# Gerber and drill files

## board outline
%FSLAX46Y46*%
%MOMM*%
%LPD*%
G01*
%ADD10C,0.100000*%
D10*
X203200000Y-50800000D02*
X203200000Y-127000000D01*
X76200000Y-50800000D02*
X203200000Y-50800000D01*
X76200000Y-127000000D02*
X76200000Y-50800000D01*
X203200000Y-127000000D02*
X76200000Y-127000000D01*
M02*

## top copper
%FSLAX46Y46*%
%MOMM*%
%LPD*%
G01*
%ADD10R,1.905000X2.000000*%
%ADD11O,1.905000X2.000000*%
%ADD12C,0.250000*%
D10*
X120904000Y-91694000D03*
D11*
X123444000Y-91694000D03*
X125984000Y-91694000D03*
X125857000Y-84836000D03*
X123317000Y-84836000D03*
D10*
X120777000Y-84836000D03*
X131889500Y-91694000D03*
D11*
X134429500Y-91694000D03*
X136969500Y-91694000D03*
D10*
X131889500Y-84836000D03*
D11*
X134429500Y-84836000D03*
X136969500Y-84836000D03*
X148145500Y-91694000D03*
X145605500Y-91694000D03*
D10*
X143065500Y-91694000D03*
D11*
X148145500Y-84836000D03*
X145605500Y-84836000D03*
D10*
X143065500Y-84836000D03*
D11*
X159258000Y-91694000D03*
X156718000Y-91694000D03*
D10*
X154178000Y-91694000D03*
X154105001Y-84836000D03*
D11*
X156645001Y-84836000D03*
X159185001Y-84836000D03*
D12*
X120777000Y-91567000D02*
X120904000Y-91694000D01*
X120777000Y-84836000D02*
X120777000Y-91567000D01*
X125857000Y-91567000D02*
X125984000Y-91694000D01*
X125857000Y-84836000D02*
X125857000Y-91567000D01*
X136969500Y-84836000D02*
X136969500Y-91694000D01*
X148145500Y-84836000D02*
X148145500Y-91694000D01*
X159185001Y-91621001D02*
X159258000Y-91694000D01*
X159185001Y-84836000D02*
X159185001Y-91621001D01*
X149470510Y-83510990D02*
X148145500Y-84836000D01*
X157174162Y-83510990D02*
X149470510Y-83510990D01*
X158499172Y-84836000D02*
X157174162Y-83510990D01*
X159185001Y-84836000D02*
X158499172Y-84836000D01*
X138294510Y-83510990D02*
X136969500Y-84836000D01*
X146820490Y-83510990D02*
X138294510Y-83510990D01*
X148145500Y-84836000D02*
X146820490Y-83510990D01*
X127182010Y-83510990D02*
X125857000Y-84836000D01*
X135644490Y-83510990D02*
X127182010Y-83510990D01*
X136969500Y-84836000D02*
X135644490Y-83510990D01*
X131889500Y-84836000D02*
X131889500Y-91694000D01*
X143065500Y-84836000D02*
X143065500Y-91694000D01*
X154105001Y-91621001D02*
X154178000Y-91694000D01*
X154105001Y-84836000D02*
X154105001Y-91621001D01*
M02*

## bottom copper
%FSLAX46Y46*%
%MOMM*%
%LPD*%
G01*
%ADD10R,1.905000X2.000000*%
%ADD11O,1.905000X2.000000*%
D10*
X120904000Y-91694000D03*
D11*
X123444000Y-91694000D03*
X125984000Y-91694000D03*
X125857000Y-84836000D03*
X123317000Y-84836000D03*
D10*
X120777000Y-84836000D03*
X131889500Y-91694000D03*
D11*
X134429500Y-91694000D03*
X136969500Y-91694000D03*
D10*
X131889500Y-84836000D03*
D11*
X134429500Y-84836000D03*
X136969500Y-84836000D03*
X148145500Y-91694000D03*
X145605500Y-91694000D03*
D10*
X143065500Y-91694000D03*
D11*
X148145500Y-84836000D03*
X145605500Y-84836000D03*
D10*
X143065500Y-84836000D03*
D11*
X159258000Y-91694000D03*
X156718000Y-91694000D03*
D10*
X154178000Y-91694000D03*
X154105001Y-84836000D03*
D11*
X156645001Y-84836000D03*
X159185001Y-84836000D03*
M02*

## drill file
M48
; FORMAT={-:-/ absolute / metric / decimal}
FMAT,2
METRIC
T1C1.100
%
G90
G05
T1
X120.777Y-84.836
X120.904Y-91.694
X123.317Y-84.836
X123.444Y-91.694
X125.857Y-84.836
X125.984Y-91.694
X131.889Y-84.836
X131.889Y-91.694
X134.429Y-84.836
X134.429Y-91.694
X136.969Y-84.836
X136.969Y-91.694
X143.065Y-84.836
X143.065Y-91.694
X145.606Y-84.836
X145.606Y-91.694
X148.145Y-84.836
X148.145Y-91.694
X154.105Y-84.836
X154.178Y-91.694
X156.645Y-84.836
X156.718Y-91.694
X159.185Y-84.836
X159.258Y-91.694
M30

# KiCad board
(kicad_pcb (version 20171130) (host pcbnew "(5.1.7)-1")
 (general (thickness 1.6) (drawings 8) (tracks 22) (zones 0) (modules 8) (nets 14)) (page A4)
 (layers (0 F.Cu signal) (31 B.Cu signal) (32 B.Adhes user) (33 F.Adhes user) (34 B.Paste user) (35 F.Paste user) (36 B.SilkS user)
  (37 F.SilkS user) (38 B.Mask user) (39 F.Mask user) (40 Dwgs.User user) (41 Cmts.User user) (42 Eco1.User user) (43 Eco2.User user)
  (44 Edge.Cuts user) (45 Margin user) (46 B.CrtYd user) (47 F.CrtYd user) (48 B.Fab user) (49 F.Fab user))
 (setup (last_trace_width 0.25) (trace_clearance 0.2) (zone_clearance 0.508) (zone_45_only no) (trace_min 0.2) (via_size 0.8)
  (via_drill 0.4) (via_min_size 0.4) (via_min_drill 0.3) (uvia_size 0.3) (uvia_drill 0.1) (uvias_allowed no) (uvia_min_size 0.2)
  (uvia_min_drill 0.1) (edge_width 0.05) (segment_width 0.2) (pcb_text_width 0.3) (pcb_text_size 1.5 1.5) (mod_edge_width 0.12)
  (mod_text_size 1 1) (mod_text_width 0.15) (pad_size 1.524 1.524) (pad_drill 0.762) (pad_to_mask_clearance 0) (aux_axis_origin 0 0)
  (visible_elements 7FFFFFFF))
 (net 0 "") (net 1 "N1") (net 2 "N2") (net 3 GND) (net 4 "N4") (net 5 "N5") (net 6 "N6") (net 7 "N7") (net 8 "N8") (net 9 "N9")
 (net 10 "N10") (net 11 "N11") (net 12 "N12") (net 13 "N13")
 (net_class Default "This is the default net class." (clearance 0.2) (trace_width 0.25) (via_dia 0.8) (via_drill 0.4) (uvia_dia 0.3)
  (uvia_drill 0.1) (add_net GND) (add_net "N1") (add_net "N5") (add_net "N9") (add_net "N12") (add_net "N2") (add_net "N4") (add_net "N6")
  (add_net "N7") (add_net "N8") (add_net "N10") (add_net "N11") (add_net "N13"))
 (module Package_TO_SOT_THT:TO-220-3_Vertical (layer F.Cu) (at 120.904 91.694)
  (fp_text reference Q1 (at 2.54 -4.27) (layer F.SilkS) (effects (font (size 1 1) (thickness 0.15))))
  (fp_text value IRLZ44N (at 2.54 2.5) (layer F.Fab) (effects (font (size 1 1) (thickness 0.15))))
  (pad 1 thru_hole rect (at 0 0) (size 1.905 2) (drill 1.1) (layers *.Cu *.Mask) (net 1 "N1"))
  (pad 2 thru_hole oval (at 2.54 0) (size 1.905 2) (drill 1.1) (layers *.Cu *.Mask) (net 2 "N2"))
  (pad 3 thru_hole oval (at 5.08 0) (size 1.905 2) (drill 1.1) (layers *.Cu *.Mask) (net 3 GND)))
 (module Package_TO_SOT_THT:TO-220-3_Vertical (layer F.Cu) (at 120.777 84.836)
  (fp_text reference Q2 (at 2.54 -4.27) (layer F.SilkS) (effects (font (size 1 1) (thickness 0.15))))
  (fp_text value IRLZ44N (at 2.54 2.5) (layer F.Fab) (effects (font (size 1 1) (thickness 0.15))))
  (pad 3 thru_hole oval (at 5.08 0) (size 1.905 2) (drill 1.1) (layers *.Cu *.Mask) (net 3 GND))
  (pad 2 thru_hole oval (at 2.54 0) (size 1.905 2) (drill 1.1) (layers *.Cu *.Mask) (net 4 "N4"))
  (pad 1 thru_hole rect (at 0 0) (size 1.905 2) (drill 1.1) (layers *.Cu *.Mask) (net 1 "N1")))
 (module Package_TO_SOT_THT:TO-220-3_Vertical (layer F.Cu) (at 131.8895 91.694)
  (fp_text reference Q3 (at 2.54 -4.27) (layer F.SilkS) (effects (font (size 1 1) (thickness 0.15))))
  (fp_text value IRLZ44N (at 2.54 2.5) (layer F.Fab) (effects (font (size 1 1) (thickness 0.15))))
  (pad 1 thru_hole rect (at 0 0) (size 1.905 2) (drill 1.1) (layers *.Cu *.Mask) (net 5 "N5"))
  (pad 2 thru_hole oval (at 2.54 0) (size 1.905 2) (drill 1.1) (layers *.Cu *.Mask) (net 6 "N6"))
  (pad 3 thru_hole oval (at 5.08 0) (size 1.905 2) (drill 1.1) (layers *.Cu *.Mask) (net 3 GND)))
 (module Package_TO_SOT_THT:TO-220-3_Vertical (layer F.Cu) (at 131.8895 84.836)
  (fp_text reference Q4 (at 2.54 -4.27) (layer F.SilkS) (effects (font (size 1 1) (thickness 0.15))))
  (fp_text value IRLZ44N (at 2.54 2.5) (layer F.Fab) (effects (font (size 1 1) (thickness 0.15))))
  (pad 1 thru_hole rect (at 0 0) (size 1.905 2) (drill 1.1) (layers *.Cu *.Mask) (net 5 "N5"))
  (pad 2 thru_hole oval (at 2.54 0) (size 1.905 2) (drill 1.1) (layers *.Cu *.Mask) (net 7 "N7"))
  (pad 3 thru_hole oval (at 5.08 0) (size 1.905 2) (drill 1.1) (layers *.Cu *.Mask) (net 3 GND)))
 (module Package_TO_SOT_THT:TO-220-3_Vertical (layer F.Cu) (at 143.0655 91.694)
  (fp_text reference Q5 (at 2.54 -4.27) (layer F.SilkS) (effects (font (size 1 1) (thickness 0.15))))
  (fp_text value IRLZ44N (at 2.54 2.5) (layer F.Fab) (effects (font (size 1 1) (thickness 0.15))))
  (pad 3 thru_hole oval (at 5.08 0) (size 1.905 2) (drill 1.1) (layers *.Cu *.Mask) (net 3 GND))
  (pad 2 thru_hole oval (at 2.54 0) (size 1.905 2) (drill 1.1) (layers *.Cu *.Mask) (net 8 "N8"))
  (pad 1 thru_hole rect (at 0 0) (size 1.905 2) (drill 1.1) (layers *.Cu *.Mask) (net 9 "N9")))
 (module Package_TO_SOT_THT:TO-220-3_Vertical (layer F.Cu) (at 143.0655 84.836)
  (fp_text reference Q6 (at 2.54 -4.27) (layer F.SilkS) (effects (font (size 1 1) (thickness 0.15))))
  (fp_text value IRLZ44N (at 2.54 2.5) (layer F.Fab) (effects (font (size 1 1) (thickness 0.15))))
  (pad 3 thru_hole oval (at 5.08 0) (size 1.905 2) (drill 1.1) (layers *.Cu *.Mask) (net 3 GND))
  (pad 2 thru_hole oval (at 2.54 0) (size 1.905 2) (drill 1.1) (layers *.Cu *.Mask) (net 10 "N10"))
  (pad 1 thru_hole rect (at 0 0) (size 1.905 2) (drill 1.1) (layers *.Cu *.Mask) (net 9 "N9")))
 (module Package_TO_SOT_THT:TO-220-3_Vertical (layer F.Cu) (at 154.178 91.694)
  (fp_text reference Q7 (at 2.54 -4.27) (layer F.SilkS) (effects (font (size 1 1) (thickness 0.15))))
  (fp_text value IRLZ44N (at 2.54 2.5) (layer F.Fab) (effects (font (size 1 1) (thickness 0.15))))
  (pad 3 thru_hole oval (at 5.08 0) (size 1.905 2) (drill 1.1) (layers *.Cu *.Mask) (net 3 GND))
  (pad 2 thru_hole oval (at 2.54 0) (size 1.905 2) (drill 1.1) (layers *.Cu *.Mask) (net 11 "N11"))
  (pad 1 thru_hole rect (at 0 0) (size 1.905 2) (drill 1.1) (layers *.Cu *.Mask) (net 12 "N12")))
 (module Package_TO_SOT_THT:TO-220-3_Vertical (layer F.Cu) (at 154.105001 84.836)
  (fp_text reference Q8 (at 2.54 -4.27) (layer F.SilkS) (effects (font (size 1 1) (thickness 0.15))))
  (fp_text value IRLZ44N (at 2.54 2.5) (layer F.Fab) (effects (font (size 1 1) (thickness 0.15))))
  (pad 1 thru_hole rect (at 0 0) (size 1.905 2) (drill 1.1) (layers *.Cu *.Mask) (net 12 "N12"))
  (pad 2 thru_hole oval (at 2.54 0) (size 1.905 2) (drill 1.1) (layers *.Cu *.Mask) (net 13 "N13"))
  (pad 3 thru_hole oval (at 5.08 0) (size 1.905 2) (drill 1.1) (layers *.Cu *.Mask) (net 3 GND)))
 (gr_line (start 203.2 50.8) (end 203.2 127) (layer Edge.Cuts) (width 0.1))
 (gr_line (start 76.2 50.8) (end 203.2 50.8) (layer Edge.Cuts) (width 0.1))
 (gr_line (start 76.2 127) (end 76.2 50.8) (layer Edge.Cuts) (width 0.1))
 (gr_line (start 203.2 127) (end 76.2 127) (layer Edge.Cuts) (width 0.1))
 (segment (start 120.777 91.567) (end 120.904 91.694) (width 0.25) (layer F.Cu) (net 1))
 (segment (start 120.777 84.836) (end 120.777 91.567) (width 0.25) (layer F.Cu) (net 1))
 (segment (start 125.857 91.567) (end 125.984 91.694) (width 0.25) (layer F.Cu) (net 3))
 (segment (start 125.857 84.836) (end 125.857 91.567) (width 0.25) (layer F.Cu) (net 3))
 (segment (start 136.9695 84.836) (end 136.9695 91.694) (width 0.25) (layer F.Cu) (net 3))
 (segment (start 148.1455 84.836) (end 148.1455 91.694) (width 0.25) (layer F.Cu) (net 3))
 (segment (start 159.185001 91.621001) (end 159.258 91.694) (width 0.25) (layer F.Cu) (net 3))
 (segment (start 159.185001 84.836) (end 159.185001 91.621001) (width 0.25) (layer F.Cu) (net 3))
 (segment (start 149.47051 83.51099) (end 148.1455 84.836) (width 0.25) (layer F.Cu) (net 3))
 (segment (start 157.174162 83.51099) (end 149.47051 83.51099) (width 0.25) (layer F.Cu) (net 3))
 (segment (start 158.499172 84.836) (end 157.174162 83.51099) (width 0.25) (layer F.Cu) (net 3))
 (segment (start 159.185001 84.836) (end 158.499172 84.836) (width 0.25) (layer F.Cu) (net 3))
 (segment (start 138.29451 83.51099) (end 136.9695 84.836) (width 0.25) (layer F.Cu) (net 3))
 (segment (start 146.82049 83.51099) (end 138.29451 83.51099) (width 0.25) (layer F.Cu) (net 3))
 (segment (start 148.1455 84.836) (end 146.82049 83.51099) (width 0.25) (layer F.Cu) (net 3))
 (segment (start 127.18201 83.51099) (end 125.857 84.836) (width 0.25) (layer F.Cu) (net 3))
 (segment (start 135.64449 83.51099) (end 127.18201 83.51099) (width 0.25) (layer F.Cu) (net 3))
 (segment (start 136.9695 84.836) (end 135.64449 83.51099) (width 0.25) (layer F.Cu) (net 3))
 (segment (start 131.8895 84.836) (end 131.8895 91.694) (width 0.25) (layer F.Cu) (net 5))
 (segment (start 143.0655 84.836) (end 143.0655 91.694) (width 0.25) (layer F.Cu) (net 9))
 (segment (start 154.105001 91.621001) (end 154.178 91.694) (width 0.25) (layer F.Cu) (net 12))
 (segment (start 154.105001 84.836) (end 154.105001 91.621001) (width 0.25) (layer F.Cu) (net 12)))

